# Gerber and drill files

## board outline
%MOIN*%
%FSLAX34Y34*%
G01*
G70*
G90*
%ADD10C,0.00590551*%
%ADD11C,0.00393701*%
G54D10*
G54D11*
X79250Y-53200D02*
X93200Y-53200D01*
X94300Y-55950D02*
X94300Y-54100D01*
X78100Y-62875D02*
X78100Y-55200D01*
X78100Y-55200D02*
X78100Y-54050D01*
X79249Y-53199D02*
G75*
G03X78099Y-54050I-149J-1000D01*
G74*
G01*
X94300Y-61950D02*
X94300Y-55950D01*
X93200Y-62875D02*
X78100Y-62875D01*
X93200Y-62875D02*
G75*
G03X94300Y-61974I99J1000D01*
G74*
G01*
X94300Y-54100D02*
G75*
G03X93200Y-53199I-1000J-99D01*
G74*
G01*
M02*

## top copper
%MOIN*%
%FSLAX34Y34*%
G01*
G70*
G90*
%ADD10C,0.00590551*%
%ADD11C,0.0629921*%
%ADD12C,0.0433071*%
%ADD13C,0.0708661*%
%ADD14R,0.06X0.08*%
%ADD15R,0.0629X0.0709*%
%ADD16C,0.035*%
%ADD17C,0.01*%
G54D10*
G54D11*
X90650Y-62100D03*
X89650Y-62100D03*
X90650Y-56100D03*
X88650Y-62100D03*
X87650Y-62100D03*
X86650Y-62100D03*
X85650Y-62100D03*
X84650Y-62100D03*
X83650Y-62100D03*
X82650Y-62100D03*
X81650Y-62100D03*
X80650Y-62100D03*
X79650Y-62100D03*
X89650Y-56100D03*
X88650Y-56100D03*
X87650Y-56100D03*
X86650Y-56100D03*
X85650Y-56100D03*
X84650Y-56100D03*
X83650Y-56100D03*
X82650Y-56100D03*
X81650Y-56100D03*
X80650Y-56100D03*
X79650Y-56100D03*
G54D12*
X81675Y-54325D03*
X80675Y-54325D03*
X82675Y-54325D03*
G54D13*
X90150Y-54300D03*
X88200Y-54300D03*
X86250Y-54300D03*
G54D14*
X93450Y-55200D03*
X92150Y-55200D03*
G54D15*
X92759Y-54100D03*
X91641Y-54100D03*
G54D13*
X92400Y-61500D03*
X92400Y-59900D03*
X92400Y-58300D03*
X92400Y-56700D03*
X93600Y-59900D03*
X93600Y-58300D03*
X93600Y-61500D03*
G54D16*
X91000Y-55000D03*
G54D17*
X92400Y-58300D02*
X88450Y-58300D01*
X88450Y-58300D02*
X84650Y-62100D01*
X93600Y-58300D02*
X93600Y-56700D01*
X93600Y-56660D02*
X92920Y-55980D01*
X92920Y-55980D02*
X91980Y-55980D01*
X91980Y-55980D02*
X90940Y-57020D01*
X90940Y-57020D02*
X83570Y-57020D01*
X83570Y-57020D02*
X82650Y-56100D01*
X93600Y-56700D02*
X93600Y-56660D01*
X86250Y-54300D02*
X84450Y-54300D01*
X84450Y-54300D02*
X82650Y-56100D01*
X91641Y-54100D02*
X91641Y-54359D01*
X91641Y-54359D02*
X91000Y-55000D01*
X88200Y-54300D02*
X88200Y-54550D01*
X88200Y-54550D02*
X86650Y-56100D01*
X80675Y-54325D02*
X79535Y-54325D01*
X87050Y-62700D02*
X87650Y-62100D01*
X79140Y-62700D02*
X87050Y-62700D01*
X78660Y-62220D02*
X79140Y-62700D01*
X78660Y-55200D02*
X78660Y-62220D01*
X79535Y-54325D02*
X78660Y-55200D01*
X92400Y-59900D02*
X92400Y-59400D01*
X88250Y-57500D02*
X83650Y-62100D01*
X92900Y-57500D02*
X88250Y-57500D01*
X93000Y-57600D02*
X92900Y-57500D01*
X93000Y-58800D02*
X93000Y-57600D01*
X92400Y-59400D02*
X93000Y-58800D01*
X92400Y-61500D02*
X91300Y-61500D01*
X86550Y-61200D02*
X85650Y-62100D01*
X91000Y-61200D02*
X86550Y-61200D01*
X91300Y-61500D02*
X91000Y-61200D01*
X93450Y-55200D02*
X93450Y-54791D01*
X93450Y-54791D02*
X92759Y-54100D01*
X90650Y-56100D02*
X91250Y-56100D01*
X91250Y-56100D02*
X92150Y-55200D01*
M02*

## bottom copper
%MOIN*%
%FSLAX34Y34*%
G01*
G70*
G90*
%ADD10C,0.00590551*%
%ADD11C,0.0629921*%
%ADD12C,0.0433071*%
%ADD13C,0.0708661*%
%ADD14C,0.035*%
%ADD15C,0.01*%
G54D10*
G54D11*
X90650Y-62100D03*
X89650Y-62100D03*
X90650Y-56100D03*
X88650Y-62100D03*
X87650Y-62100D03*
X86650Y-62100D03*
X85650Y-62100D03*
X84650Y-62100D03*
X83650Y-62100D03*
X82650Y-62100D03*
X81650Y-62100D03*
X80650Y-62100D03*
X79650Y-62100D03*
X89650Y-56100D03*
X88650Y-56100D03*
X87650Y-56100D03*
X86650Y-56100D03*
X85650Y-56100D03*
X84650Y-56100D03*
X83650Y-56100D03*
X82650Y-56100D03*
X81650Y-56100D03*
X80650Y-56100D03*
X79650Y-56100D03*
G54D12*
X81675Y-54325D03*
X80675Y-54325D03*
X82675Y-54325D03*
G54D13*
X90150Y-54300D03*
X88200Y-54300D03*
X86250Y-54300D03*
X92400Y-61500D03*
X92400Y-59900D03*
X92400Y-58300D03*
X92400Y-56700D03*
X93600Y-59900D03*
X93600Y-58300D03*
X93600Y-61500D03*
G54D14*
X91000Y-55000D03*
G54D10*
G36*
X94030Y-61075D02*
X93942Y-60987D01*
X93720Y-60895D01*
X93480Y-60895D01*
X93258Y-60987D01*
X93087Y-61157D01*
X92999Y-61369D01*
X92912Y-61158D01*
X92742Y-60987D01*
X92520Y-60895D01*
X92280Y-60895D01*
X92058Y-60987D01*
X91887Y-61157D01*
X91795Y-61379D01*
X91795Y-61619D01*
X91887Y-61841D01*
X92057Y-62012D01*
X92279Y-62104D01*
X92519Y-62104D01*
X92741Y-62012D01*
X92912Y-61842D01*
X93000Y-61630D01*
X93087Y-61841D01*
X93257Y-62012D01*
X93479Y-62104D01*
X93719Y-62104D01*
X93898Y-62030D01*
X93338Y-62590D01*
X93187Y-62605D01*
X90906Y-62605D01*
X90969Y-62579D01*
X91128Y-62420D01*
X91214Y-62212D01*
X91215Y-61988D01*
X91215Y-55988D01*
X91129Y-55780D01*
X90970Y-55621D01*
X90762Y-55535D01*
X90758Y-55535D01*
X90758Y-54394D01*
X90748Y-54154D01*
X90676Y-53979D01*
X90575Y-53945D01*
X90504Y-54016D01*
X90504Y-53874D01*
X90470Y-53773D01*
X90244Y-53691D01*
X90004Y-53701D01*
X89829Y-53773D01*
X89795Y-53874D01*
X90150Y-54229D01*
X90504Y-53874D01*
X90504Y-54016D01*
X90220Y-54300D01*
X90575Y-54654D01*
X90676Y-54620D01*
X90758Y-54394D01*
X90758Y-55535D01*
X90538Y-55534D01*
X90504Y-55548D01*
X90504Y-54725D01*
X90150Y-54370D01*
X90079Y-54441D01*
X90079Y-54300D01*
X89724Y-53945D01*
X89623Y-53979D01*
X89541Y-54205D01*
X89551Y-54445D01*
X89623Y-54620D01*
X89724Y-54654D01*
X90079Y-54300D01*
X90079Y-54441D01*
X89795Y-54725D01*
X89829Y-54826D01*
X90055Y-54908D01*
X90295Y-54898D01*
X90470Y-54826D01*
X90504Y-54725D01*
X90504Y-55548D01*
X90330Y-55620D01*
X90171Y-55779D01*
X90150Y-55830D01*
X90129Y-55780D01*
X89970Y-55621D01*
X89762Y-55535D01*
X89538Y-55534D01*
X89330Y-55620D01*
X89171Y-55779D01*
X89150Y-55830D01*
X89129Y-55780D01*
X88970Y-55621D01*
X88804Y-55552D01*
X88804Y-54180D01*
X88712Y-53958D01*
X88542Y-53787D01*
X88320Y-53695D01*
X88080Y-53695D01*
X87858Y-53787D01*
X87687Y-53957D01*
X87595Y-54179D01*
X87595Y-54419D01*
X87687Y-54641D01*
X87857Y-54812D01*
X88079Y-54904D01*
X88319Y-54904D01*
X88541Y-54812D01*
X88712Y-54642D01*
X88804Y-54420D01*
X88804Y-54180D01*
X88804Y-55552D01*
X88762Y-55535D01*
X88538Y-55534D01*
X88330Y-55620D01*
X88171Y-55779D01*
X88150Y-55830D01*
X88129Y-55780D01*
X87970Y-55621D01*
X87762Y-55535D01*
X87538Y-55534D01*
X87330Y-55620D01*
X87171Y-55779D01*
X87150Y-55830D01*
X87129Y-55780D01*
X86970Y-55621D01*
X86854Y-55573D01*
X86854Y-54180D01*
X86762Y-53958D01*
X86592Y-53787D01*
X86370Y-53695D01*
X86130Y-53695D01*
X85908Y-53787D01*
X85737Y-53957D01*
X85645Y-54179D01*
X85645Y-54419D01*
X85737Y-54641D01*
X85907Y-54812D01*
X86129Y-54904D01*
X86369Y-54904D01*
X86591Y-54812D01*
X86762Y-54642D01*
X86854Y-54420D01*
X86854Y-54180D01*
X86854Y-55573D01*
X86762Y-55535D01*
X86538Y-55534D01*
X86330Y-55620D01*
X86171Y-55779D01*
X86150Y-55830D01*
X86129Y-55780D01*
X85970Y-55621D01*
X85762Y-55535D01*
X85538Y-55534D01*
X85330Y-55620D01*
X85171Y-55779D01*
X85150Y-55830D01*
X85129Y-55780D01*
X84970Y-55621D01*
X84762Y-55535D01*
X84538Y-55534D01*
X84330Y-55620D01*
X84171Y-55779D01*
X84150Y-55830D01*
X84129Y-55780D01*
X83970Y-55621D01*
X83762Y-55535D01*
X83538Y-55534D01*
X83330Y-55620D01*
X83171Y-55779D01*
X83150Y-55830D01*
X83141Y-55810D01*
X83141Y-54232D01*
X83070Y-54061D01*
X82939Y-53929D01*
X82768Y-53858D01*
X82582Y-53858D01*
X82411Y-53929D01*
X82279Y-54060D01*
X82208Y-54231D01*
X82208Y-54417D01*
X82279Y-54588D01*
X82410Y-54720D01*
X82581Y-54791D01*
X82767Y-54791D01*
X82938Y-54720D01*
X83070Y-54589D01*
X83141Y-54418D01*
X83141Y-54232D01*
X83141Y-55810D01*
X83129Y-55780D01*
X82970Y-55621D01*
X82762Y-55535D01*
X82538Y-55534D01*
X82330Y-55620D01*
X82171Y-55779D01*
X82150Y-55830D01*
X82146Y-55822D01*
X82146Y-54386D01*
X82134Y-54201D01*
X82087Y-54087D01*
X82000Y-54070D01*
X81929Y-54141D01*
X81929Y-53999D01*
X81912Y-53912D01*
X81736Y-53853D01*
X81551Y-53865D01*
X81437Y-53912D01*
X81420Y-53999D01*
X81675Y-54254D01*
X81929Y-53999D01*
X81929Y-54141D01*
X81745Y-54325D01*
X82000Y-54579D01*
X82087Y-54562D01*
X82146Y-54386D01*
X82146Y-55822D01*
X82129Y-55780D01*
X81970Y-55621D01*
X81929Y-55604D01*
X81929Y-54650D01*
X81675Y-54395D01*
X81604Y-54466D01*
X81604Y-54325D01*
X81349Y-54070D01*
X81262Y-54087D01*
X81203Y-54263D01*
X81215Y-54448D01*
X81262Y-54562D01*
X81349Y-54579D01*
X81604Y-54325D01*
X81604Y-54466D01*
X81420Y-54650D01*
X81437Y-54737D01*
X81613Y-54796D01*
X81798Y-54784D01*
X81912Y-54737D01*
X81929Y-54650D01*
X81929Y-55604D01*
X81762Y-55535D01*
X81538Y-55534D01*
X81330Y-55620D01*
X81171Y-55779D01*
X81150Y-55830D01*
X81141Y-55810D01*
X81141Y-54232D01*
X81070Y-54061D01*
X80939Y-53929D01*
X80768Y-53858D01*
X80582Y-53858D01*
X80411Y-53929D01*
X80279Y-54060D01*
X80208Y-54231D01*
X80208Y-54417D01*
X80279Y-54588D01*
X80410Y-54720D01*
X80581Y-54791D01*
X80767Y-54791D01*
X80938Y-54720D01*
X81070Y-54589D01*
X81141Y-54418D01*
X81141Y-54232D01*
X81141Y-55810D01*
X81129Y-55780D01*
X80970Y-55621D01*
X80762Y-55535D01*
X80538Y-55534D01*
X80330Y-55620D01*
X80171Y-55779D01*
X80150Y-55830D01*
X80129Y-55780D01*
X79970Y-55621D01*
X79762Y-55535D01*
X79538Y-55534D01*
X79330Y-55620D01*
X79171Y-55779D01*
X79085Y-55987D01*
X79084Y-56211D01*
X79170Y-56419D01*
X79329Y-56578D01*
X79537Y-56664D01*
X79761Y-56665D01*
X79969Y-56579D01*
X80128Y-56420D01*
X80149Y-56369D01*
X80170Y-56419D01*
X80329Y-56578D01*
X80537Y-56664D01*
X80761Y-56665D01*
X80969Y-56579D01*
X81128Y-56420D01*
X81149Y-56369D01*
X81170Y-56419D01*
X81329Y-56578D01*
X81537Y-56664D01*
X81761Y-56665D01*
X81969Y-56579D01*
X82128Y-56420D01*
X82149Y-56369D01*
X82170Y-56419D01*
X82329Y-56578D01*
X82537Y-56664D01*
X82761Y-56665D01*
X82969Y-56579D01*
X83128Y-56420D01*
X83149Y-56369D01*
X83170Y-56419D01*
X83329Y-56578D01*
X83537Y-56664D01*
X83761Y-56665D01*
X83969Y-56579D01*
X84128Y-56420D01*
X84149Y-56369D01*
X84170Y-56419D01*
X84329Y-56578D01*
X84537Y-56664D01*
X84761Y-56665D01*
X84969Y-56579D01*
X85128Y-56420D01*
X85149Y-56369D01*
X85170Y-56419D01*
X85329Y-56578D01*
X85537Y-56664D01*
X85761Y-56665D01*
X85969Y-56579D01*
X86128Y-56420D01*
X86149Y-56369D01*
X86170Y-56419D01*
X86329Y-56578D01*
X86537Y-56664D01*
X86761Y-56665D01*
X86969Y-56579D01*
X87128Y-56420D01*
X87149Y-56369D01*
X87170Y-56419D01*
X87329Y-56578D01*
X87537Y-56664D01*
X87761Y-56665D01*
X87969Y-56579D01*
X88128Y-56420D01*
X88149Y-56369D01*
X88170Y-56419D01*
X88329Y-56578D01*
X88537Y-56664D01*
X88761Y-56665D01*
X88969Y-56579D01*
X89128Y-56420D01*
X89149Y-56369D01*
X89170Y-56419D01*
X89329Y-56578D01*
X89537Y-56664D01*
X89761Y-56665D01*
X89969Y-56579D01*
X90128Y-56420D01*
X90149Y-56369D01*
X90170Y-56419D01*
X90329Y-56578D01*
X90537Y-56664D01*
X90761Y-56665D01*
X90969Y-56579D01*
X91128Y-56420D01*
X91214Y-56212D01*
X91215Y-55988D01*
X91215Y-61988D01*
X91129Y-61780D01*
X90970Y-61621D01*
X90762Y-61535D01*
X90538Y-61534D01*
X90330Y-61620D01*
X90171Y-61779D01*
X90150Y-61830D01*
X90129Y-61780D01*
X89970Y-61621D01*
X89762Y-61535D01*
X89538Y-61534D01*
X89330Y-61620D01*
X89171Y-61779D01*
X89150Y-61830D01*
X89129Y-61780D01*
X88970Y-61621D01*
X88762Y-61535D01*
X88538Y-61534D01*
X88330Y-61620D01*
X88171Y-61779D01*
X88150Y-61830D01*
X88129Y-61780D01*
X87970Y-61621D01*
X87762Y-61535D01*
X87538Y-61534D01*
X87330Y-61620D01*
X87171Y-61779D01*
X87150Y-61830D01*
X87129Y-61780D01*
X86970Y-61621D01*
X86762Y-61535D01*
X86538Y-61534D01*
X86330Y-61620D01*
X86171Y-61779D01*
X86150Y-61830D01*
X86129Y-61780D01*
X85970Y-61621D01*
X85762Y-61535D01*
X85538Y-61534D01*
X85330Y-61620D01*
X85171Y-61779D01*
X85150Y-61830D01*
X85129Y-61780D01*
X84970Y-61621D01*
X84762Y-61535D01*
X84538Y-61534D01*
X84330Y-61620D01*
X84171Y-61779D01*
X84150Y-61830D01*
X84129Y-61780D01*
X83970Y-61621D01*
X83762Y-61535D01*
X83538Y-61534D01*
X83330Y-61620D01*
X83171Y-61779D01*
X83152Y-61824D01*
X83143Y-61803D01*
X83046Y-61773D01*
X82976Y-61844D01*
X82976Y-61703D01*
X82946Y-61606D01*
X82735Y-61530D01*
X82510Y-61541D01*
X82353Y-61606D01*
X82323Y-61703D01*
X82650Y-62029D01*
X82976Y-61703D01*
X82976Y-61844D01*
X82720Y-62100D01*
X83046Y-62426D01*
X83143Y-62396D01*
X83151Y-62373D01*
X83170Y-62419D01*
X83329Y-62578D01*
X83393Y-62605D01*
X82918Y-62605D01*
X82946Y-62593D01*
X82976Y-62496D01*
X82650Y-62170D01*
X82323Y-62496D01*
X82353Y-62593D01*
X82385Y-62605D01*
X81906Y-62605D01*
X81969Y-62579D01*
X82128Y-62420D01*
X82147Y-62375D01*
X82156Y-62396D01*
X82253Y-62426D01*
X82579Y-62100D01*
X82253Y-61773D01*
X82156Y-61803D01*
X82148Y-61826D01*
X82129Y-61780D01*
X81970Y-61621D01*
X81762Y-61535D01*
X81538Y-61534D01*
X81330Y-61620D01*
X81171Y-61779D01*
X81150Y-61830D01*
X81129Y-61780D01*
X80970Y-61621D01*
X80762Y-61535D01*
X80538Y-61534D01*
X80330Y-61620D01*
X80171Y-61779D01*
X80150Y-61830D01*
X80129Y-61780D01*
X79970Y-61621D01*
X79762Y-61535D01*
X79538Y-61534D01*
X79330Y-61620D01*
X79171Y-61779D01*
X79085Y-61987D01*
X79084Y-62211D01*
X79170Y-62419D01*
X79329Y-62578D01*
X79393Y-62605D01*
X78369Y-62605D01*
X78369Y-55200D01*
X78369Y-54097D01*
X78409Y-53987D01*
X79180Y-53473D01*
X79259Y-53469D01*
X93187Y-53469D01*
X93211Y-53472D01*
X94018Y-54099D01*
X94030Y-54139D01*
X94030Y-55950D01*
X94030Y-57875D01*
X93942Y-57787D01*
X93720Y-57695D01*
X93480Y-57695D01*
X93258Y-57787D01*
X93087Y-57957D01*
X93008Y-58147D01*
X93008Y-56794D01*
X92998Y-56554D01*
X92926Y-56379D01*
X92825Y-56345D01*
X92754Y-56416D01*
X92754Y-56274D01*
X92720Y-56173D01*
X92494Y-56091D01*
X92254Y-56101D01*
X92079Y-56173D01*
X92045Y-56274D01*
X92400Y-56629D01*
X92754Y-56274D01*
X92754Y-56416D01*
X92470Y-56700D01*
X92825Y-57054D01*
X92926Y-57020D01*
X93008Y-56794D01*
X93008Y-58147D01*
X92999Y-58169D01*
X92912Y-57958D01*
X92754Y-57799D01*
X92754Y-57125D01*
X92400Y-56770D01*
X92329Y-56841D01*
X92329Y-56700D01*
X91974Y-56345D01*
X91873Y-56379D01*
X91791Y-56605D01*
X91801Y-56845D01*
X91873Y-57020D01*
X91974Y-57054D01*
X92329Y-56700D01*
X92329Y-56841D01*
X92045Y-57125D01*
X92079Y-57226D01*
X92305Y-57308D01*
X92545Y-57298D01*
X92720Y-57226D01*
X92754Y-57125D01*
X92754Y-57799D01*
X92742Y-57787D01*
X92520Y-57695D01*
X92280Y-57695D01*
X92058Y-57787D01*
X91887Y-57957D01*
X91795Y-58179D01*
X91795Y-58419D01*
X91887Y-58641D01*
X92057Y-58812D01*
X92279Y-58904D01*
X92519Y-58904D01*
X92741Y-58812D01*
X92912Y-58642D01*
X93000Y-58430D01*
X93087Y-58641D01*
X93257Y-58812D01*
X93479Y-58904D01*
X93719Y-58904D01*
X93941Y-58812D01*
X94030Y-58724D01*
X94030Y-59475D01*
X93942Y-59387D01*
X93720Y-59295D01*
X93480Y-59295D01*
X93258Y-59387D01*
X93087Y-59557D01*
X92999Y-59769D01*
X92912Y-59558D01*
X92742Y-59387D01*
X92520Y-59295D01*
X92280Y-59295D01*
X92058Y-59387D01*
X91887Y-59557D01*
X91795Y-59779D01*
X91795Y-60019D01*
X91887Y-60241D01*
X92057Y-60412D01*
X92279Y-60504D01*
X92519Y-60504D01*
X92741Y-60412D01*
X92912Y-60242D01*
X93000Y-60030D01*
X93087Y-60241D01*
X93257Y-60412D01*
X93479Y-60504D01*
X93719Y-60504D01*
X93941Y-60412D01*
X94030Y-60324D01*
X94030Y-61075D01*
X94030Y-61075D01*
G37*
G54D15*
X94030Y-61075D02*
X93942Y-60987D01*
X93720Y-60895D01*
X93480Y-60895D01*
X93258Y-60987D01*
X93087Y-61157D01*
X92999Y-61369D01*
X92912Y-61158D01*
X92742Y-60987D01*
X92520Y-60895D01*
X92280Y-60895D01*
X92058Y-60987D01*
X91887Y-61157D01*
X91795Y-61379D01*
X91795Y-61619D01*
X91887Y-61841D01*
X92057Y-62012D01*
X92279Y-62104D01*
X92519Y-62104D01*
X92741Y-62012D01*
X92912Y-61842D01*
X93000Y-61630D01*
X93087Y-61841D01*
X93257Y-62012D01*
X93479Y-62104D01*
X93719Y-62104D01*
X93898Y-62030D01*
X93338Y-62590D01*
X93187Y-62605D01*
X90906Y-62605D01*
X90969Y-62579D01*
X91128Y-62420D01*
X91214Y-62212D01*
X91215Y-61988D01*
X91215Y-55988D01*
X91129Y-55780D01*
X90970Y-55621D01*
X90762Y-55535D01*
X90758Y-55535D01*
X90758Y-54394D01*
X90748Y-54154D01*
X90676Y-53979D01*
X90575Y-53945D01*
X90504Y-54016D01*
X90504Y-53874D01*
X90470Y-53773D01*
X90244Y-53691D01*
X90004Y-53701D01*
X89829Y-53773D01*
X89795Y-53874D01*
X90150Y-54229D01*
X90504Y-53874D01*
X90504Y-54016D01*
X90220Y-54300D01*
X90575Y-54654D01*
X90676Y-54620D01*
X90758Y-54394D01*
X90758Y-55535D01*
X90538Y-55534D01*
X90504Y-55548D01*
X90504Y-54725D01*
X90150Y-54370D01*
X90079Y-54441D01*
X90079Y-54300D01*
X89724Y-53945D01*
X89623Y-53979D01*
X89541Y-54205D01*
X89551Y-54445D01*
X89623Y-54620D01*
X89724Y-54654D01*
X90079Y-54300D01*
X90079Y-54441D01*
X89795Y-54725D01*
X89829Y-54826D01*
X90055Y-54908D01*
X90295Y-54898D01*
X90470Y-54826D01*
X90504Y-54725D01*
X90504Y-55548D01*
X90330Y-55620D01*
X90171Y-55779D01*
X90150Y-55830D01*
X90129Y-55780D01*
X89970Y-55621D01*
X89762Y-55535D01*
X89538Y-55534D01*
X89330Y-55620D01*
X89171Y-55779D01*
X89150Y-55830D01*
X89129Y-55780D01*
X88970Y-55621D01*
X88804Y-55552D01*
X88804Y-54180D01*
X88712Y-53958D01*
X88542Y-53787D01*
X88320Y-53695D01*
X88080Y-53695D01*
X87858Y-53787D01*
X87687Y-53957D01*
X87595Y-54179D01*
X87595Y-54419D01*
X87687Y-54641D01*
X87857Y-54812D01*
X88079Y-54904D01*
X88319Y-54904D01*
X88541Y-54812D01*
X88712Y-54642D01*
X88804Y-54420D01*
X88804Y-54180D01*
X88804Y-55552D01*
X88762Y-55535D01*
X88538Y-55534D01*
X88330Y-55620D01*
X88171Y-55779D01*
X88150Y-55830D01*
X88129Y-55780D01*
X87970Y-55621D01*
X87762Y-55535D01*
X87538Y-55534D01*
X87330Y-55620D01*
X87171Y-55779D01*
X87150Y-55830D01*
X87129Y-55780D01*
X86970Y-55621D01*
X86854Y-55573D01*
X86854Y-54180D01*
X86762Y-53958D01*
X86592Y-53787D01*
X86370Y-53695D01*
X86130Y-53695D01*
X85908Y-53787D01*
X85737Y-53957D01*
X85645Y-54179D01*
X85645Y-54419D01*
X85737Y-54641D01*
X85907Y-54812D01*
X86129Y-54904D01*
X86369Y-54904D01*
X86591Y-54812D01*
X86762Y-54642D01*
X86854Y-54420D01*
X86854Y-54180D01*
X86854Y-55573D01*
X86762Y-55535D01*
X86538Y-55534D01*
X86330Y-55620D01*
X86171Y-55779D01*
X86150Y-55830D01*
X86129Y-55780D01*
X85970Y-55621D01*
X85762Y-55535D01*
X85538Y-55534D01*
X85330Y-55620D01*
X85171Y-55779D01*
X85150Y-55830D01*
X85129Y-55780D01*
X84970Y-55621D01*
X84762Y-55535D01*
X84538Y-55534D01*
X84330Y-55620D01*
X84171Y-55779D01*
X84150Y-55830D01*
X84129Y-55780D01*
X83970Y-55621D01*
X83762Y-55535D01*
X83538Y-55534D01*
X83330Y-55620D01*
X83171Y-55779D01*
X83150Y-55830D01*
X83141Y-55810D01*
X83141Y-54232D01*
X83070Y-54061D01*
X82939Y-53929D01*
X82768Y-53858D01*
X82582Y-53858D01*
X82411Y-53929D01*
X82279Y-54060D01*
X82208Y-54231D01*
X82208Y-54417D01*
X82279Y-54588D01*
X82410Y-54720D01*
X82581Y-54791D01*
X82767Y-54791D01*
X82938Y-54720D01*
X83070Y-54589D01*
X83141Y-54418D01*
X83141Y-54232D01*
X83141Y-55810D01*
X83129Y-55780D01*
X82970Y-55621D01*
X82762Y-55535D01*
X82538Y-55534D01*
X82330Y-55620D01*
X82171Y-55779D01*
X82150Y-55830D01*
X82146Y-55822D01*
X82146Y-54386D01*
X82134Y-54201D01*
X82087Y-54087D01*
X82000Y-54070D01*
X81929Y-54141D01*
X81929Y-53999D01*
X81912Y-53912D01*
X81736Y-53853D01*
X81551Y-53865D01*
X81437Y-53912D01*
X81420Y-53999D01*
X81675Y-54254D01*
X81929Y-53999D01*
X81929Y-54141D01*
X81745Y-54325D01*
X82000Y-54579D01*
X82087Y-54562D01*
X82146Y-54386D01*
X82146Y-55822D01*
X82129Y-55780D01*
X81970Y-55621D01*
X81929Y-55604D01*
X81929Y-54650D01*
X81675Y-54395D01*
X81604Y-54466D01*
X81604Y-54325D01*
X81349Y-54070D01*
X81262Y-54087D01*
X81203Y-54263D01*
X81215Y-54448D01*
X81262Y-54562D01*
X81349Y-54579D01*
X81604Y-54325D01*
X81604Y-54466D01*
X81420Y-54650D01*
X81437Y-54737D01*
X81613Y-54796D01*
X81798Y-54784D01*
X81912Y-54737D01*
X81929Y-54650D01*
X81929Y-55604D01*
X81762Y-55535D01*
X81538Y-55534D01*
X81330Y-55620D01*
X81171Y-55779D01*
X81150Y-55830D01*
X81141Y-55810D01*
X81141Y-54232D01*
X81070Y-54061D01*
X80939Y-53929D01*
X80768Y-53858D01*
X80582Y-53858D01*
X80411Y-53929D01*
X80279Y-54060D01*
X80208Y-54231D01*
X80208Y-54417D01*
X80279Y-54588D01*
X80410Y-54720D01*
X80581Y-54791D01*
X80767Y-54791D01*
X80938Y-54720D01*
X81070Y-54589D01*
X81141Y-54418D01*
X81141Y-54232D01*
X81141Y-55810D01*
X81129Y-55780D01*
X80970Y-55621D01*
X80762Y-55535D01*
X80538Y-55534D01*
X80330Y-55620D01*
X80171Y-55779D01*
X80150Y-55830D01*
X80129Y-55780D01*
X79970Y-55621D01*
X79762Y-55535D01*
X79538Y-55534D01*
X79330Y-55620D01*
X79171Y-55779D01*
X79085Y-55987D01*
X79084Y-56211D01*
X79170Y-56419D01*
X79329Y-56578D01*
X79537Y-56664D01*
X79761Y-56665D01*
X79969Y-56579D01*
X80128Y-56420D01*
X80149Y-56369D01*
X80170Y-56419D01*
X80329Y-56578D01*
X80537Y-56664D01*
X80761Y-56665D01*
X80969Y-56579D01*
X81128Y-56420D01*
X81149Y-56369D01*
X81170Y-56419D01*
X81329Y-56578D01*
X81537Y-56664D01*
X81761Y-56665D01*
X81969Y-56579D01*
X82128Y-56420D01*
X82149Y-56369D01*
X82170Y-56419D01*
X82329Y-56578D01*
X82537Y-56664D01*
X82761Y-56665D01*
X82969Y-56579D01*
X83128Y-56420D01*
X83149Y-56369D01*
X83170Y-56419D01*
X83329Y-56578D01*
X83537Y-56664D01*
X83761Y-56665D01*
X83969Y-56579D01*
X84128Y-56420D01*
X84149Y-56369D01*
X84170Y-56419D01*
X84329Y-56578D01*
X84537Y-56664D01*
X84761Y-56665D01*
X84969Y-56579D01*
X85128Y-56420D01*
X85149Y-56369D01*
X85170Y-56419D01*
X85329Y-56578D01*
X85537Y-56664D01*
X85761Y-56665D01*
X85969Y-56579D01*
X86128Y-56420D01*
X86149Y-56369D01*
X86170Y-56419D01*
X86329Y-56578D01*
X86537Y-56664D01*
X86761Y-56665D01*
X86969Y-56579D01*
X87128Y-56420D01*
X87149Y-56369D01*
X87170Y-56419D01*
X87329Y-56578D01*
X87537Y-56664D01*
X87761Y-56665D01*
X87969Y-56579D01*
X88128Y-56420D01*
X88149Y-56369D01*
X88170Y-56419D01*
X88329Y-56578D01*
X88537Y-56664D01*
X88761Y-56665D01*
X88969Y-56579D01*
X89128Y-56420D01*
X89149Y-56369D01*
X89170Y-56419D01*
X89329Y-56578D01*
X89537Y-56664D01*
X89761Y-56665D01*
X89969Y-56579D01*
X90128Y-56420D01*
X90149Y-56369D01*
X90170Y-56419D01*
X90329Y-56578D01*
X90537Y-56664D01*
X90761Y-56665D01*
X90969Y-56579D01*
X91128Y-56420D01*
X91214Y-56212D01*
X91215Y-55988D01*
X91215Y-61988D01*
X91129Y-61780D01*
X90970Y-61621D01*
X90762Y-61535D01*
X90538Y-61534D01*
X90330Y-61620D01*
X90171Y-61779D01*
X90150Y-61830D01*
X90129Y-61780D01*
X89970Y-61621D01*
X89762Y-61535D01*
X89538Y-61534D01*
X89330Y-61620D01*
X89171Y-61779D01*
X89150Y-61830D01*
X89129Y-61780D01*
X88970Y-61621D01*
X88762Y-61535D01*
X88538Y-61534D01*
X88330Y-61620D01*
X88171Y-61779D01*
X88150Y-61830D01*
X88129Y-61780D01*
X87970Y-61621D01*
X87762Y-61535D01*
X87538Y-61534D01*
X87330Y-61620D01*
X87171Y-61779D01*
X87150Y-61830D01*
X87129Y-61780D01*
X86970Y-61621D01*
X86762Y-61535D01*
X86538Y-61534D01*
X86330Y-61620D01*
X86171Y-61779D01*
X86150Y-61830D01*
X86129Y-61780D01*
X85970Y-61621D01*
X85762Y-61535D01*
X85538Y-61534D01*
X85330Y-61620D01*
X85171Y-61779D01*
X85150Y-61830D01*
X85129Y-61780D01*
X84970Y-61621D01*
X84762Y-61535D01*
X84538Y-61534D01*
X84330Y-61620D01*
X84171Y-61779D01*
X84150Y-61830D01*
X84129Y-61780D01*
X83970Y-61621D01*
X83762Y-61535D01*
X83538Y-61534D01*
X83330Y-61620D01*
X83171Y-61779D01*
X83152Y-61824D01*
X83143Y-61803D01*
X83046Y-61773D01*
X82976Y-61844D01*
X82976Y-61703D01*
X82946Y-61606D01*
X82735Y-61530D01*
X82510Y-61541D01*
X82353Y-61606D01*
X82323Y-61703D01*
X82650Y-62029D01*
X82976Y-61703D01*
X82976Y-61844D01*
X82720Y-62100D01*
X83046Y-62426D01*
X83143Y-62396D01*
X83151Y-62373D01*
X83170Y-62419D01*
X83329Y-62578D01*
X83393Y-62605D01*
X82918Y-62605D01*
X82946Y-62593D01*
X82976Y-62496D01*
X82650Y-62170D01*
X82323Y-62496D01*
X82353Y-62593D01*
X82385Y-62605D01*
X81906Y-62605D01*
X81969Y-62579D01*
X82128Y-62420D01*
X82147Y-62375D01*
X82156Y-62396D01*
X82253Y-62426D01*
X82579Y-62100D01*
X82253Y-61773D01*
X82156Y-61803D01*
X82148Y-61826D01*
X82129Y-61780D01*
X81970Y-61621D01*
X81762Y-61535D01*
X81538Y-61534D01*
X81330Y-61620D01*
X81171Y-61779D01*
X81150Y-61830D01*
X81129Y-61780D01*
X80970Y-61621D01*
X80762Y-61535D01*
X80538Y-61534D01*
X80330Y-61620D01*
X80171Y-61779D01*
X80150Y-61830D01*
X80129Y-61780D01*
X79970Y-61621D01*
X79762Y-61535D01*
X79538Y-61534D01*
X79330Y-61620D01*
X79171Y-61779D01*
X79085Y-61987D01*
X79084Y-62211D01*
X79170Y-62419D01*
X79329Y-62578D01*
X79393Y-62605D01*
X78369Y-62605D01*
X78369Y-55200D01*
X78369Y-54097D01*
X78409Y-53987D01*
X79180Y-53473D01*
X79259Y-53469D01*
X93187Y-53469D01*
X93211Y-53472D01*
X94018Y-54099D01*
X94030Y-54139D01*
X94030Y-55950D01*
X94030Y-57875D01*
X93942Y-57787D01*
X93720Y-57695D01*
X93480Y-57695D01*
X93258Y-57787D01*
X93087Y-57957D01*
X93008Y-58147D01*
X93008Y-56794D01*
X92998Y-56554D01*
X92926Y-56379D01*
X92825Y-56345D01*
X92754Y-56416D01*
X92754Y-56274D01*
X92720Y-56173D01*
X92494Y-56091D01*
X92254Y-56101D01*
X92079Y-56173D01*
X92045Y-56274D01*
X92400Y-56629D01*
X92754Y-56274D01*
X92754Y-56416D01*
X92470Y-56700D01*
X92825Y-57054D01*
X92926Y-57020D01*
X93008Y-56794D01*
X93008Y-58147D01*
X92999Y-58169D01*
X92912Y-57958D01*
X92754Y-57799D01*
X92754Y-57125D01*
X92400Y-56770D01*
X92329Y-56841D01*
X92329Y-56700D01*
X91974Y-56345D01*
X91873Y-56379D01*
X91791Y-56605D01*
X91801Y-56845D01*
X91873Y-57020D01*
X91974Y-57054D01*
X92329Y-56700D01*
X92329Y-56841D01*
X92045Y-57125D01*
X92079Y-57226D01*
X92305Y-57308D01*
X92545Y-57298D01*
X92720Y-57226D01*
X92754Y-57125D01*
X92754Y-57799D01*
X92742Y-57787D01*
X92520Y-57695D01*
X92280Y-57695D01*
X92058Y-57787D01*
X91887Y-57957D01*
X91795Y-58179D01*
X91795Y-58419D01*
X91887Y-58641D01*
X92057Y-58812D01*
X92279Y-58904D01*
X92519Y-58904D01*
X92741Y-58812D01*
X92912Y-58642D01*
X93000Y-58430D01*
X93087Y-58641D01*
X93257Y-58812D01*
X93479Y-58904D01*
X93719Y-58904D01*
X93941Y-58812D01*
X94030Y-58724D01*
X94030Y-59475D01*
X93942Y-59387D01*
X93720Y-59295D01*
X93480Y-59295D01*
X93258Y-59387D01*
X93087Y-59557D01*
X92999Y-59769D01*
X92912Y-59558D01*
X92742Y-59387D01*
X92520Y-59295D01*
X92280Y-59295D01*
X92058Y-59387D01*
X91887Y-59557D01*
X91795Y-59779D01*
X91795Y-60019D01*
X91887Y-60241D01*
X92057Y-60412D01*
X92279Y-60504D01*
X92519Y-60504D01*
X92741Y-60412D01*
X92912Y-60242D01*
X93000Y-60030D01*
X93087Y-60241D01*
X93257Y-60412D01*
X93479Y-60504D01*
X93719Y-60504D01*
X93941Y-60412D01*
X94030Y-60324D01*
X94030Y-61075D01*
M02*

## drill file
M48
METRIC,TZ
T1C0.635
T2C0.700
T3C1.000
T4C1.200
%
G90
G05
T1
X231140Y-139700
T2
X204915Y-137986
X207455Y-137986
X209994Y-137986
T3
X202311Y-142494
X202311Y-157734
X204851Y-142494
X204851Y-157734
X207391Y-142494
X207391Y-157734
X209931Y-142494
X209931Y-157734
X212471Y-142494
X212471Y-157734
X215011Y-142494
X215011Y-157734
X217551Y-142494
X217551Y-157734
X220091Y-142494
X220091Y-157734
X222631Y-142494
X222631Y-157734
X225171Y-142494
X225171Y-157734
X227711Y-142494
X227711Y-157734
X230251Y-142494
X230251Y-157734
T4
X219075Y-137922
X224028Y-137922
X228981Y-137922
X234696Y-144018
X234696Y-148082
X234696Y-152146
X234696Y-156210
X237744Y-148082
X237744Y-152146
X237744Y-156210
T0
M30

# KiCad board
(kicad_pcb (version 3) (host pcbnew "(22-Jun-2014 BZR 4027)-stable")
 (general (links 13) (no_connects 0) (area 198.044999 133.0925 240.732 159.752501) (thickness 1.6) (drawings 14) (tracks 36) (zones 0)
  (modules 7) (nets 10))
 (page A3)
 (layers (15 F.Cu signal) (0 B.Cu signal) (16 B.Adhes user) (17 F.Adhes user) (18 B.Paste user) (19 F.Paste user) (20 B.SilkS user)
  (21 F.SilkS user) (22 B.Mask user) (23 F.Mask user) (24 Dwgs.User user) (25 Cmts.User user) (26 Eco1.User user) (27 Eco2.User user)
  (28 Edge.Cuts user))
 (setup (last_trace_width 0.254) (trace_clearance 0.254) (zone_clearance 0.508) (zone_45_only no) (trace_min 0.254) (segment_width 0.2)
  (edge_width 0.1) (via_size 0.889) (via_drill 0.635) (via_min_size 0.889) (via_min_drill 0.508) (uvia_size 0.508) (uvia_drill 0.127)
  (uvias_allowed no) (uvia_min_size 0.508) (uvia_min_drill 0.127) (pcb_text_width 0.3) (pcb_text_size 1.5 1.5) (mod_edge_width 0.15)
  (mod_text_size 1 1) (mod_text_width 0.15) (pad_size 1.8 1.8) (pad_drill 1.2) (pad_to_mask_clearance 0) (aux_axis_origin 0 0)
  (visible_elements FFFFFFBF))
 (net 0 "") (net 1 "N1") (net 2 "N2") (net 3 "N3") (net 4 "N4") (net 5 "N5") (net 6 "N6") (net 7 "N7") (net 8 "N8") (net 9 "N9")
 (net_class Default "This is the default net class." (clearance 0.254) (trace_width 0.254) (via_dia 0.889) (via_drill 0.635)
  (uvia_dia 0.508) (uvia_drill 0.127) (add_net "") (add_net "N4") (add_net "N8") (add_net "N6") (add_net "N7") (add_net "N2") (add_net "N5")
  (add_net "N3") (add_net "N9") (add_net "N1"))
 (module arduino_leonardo (layer F.Cu) (at 215.138 150.114 90)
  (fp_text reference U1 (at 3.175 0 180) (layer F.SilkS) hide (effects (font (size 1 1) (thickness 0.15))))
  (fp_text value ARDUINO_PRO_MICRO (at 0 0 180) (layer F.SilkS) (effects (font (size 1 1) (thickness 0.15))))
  (pad 12 thru_hole circle (at -7.62 15.113 90) (size 1.6 1.6) (drill 1) (layers *.Cu *.Mask F.SilkS))
  (pad 11 thru_hole circle (at -7.62 12.573 90) (size 1.6 1.6) (drill 1) (layers *.Cu *.Mask F.SilkS))
  (pad 13 thru_hole circle (at 7.62 15.113 90) (size 1.6 1.6) (drill 1) (layers *.Cu *.Mask F.SilkS) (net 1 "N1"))
  (pad 10 thru_hole circle (at -7.62 10.033 90) (size 1.6 1.6) (drill 1) (layers *.Cu *.Mask F.SilkS))
  (pad 9 thru_hole circle (at -7.62 7.493 90) (size 1.6 1.6) (drill 1) (layers *.Cu *.Mask F.SilkS) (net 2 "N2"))
  (pad 8 thru_hole circle (at -7.62 4.953 90) (size 1.6 1.6) (drill 1) (layers *.Cu *.Mask F.SilkS))
  (pad 7 thru_hole circle (at -7.62 2.413 90) (size 1.6 1.6) (drill 1) (layers *.Cu *.Mask F.SilkS) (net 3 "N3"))
  (pad 6 thru_hole circle (at -7.62 -0.127 90) (size 1.6 1.6) (drill 1) (layers *.Cu *.Mask F.SilkS) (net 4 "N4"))
  (pad 5 thru_hole circle (at -7.62 -2.667 90) (size 1.6 1.6) (drill 1) (layers *.Cu *.Mask F.SilkS) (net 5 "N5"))
  (pad 4 thru_hole circle (at -7.62 -5.207 90) (size 1.6 1.6) (drill 1) (layers *.Cu *.Mask F.SilkS) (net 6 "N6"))
  (pad 3 thru_hole circle (at -7.62 -7.747 90) (size 1.6 1.6) (drill 1) (layers *.Cu *.Mask F.SilkS))
  (pad 2 thru_hole circle (at -7.62 -10.287 90) (size 1.6 1.6) (drill 1) (layers *.Cu *.Mask F.SilkS))
  (pad 1 thru_hole circle (at -7.62 -12.827 90) (size 1.6 1.6) (drill 1) (layers *.Cu *.Mask F.SilkS))
  (pad 14 thru_hole circle (at 7.62 12.573 90) (size 1.6 1.6) (drill 1) (layers *.Cu *.Mask F.SilkS))
  (pad 15 thru_hole circle (at 7.62 10.033 90) (size 1.6 1.6) (drill 1) (layers *.Cu *.Mask F.SilkS))
  (pad 16 thru_hole circle (at 7.62 7.493 90) (size 1.6 1.6) (drill 1) (layers *.Cu *.Mask F.SilkS))
  (pad 17 thru_hole circle (at 7.62 4.953 90) (size 1.6 1.6) (drill 1) (layers *.Cu *.Mask F.SilkS) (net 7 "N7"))
  (pad 18 thru_hole circle (at 7.62 2.413 90) (size 1.6 1.6) (drill 1) (layers *.Cu *.Mask F.SilkS))
  (pad 19 thru_hole circle (at 7.62 -0.127 90) (size 1.6 1.6) (drill 1) (layers *.Cu *.Mask F.SilkS))
  (pad 20 thru_hole circle (at 7.62 -2.667 90) (size 1.6 1.6) (drill 1) (layers *.Cu *.Mask F.SilkS))
  (pad 21 thru_hole circle (at 7.62 -5.207 90) (size 1.6 1.6) (drill 1) (layers *.Cu *.Mask F.SilkS) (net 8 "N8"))
  (pad 22 thru_hole circle (at 7.62 -7.747 90) (size 1.6 1.6) (drill 1) (layers *.Cu *.Mask F.SilkS))
  (pad 23 thru_hole circle (at 7.62 -10.287 90) (size 1.6 1.6) (drill 1) (layers *.Cu *.Mask F.SilkS))
  (pad 24 thru_hole circle (at 7.62 -12.827 90) (size 1.6 1.6) (drill 1) (layers *.Cu *.Mask F.SilkS)))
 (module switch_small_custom (layer F.Cu) (at 207.4545 137.9855)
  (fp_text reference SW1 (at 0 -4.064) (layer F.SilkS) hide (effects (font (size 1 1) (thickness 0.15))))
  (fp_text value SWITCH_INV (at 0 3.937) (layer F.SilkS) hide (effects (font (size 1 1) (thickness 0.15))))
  (pad 2 thru_hole circle (at 0 0) (size 1.1 1.1) (drill 0.7) (layers *.Cu *.Mask F.SilkS) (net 6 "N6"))
  (pad 1 thru_hole circle (at -2.54 0) (size 1.1 1.1) (drill 0.7) (layers *.Cu *.Mask F.SilkS) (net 2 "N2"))
  (pad 3 thru_hole circle (at 2.54 0) (size 1.1 1.1) (drill 0.7) (layers *.Cu *.Mask F.SilkS)))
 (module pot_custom (layer F.Cu) (at 224.028 137.922 180)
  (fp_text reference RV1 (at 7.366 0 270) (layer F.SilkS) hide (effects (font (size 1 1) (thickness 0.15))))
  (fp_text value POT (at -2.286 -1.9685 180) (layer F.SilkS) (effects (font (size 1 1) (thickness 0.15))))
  (pad 1 thru_hole circle (at -4.953 0 180) (size 1.8 1.8) (drill 1.2) (layers *.Cu *.Mask F.SilkS) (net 6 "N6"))
  (pad 2 thru_hole circle (at 0 0 180) (size 1.8 1.8) (drill 1.2) (layers *.Cu *.Mask F.SilkS) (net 7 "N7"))
  (pad 3 thru_hole circle (at 4.953 0 180) (size 1.8 1.8) (drill 1.2) (layers *.Cu *.Mask F.SilkS) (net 8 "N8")))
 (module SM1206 (layer F.Cu) (at 235.712 140.208 180)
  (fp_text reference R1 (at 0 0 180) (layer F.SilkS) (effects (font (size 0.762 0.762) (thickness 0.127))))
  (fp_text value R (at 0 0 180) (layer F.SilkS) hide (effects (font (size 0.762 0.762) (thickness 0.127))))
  (pad 1 smd rect (at -1.651 0 180) (size 1.524 2.032) (layers F.Cu F.Paste F.Mask) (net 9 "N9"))
  (pad 2 smd rect (at 1.651 0 180) (size 1.524 2.032) (layers F.Cu F.Paste F.Mask) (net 1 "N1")))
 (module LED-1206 (layer F.Cu) (at 234.188 137.414 180)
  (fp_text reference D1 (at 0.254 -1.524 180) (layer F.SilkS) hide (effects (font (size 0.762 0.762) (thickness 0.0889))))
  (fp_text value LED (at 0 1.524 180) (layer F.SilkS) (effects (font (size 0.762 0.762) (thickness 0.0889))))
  (pad 1 smd rect (at -1.41986 0 180) (size 1.59766 1.80086) (layers F.Cu F.Paste F.Mask) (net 9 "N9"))
  (pad 2 smd rect (at 1.41986 0 180) (size 1.59766 1.80086) (layers F.Cu F.Paste F.Mask) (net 6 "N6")))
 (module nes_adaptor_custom (layer F.Cu) (at 236.22 150.114 90)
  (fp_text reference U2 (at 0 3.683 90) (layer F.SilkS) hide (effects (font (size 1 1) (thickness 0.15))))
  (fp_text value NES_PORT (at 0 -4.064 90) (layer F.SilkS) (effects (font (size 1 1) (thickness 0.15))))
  (pad 1 thru_hole circle (at -6.096 -1.524 90) (size 1.8 1.8) (drill 1.2) (layers *.Cu *.Mask F.SilkS) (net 3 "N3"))
  (pad 2 thru_hole circle (at -2.032 -1.524 90) (size 1.8 1.8) (drill 1.2) (layers *.Cu *.Mask F.SilkS) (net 5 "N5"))
  (pad 3 thru_hole circle (at 2.032 -1.524 90) (size 1.8 1.8) (drill 1.2) (layers *.Cu *.Mask F.SilkS) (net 4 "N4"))
  (pad 4 thru_hole circle (at 6.096 -1.524 90) (size 1.8 1.8) (drill 1.2) (layers *.Cu *.Mask F.SilkS) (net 6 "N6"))
  (pad 6 thru_hole circle (at -2.032 1.524 90) (size 1.8 1.8) (drill 1.2) (layers *.Cu *.Mask F.SilkS))
  (pad 5 thru_hole circle (at 2.032 1.524 90) (size 1.8 1.8) (drill 1.2) (layers *.Cu *.Mask F.SilkS) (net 8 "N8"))
  (pad 7 thru_hole circle (at -6.096 1.524 90) (size 1.8 1.8) (drill 1.2) (layers *.Cu *.Mask F.SilkS)))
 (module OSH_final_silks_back (layer F.Cu) (at 226.949 149.225)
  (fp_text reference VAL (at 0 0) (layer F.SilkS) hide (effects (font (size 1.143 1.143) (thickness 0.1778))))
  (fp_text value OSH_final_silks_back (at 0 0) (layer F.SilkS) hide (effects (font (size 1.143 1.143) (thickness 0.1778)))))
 (gr_line (start 201.295 135.128) (end 236.728 135.128) (angle 90) (layer Edge.Cuts) (width 0.1))
 (gr_line (start 239.522 142.113) (end 239.522 137.414) (angle 90) (layer Edge.Cuts) (width 0.1))
 (gr_line (start 198.374 159.7025) (end 198.374 140.208) (angle 90) (layer Edge.Cuts) (width 0.1))
 (gr_line (start 198.374 140.208) (end 198.374 137.287) (angle 90) (layer Edge.Cuts) (width 0.1))
 (gr_arc (start 200.914 137.668) (end 198.374 137.287) (angle 90) (layer Edge.Cuts) (width 0.1))
 (gr_line (start 239.522 157.353) (end 239.522 142.113) (angle 90) (layer Edge.Cuts) (width 0.1))
 (gr_line (start 236.728 159.7025) (end 198.374 159.7025) (angle 90) (layer Edge.Cuts) (width 0.1))
 (gr_arc (start 236.982 157.1625) (end 239.522 157.4165) (angle 90) (layer Edge.Cuts) (width 0.1))
 (gr_arc (start 236.982 137.668) (end 236.728 135.128) (angle 90) (layer Edge.Cuts) (width 0.1))
 (segment (start 234.696 148.082) (end 224.663 148.082) (width 0.254) (layer F.Cu) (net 4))
 (segment (start 224.663 148.082) (end 215.011 157.734) (width 0.254) (layer F.Cu) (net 4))
 (segment (start 237.744 148.082) (end 237.744 144.018) (width 0.254) (layer F.Cu) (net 8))
 (segment (start 237.744 143.9164) (end 236.0168 142.1892) (width 0.254) (layer F.Cu) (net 8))
 (segment (start 236.0168 142.1892) (end 233.6292 142.1892) (width 0.254) (layer F.Cu) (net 8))
 (segment (start 233.6292 142.1892) (end 230.9876 144.8308) (width 0.254) (layer F.Cu) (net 8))
 (segment (start 230.9876 144.8308) (end 212.2678 144.8308) (width 0.254) (layer F.Cu) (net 8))
 (segment (start 212.2678 144.8308) (end 209.931 142.494) (width 0.254) (layer F.Cu) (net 8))
 (segment (start 237.744 144.018) (end 237.744 143.9164) (width 0.254) (layer F.Cu) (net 8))
 (segment (start 219.075 137.922) (end 214.503 137.922) (width 0.254) (layer F.Cu) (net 8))
 (segment (start 214.503 137.922) (end 209.931 142.494) (width 0.254) (layer F.Cu) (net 8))
 (segment (start 232.76814 137.414) (end 232.76814 138.07186) (width 0.254) (layer F.Cu) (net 6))
 (via (at 231.14 139.7) (size 0.889) (layers F.Cu B.Cu) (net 6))
 (segment (start 232.76814 138.07186) (end 231.14 139.7) (width 0.254) (layer F.Cu) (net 6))
 (segment (start 224.028 137.922) (end 224.028 138.557) (width 0.254) (layer F.Cu) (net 7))
 (segment (start 224.028 138.557) (end 220.091 142.494) (width 0.254) (layer F.Cu) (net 7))
 (segment (start 204.9145 137.9855) (end 202.0189 137.9855) (width 0.254) (layer F.Cu) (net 2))
 (segment (start 221.107 159.258) (end 222.631 157.734) (width 0.254) (layer F.Cu) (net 2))
 (segment (start 201.0156 159.258) (end 221.107 159.258) (width 0.254) (layer F.Cu) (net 2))
 (segment (start 199.7964 158.0388) (end 201.0156 159.258) (width 0.254) (layer F.Cu) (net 2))
 (segment (start 199.7964 140.208) (end 199.7964 158.0388) (width 0.254) (layer F.Cu) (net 2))
 (segment (start 202.0189 137.9855) (end 199.7964 140.208) (width 0.254) (layer F.Cu) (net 2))
 (segment (start 234.696 152.146) (end 234.696 150.876) (width 0.254) (layer F.Cu) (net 5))
 (segment (start 224.155 146.05) (end 212.471 157.734) (width 0.254) (layer F.Cu) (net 5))
 (segment (start 235.966 146.05) (end 224.155 146.05) (width 0.254) (layer F.Cu) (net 5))
 (segment (start 236.22 146.304) (end 235.966 146.05) (width 0.254) (layer F.Cu) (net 5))
 (segment (start 236.22 149.352) (end 236.22 146.304) (width 0.254) (layer F.Cu) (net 5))
 (segment (start 234.696 150.876) (end 236.22 149.352) (width 0.254) (layer F.Cu) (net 5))
 (segment (start 234.696 156.21) (end 231.902 156.21) (width 0.254) (layer F.Cu) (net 3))
 (segment (start 219.837 155.448) (end 217.551 157.734) (width 0.254) (layer F.Cu) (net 3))
 (segment (start 231.14 155.448) (end 219.837 155.448) (width 0.254) (layer F.Cu) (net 3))
 (segment (start 231.902 156.21) (end 231.14 155.448) (width 0.254) (layer F.Cu) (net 3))
 (segment (start 237.363 140.208) (end 237.363 139.16914) (width 0.254) (layer F.Cu) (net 9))
 (segment (start 237.363 139.16914) (end 235.60786 137.414) (width 0.254) (layer F.Cu) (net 9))
 (segment (start 230.251 142.494) (end 231.775 142.494) (width 0.254) (layer F.Cu) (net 1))
 (segment (start 231.775 142.494) (end 234.061 140.208) (width 0.254) (layer F.Cu) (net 1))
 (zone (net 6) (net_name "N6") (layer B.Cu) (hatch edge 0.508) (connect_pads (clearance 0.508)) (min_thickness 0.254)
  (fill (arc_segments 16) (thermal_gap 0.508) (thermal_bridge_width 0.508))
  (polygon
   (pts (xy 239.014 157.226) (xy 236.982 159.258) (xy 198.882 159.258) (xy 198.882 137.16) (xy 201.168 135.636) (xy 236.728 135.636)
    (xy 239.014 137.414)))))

